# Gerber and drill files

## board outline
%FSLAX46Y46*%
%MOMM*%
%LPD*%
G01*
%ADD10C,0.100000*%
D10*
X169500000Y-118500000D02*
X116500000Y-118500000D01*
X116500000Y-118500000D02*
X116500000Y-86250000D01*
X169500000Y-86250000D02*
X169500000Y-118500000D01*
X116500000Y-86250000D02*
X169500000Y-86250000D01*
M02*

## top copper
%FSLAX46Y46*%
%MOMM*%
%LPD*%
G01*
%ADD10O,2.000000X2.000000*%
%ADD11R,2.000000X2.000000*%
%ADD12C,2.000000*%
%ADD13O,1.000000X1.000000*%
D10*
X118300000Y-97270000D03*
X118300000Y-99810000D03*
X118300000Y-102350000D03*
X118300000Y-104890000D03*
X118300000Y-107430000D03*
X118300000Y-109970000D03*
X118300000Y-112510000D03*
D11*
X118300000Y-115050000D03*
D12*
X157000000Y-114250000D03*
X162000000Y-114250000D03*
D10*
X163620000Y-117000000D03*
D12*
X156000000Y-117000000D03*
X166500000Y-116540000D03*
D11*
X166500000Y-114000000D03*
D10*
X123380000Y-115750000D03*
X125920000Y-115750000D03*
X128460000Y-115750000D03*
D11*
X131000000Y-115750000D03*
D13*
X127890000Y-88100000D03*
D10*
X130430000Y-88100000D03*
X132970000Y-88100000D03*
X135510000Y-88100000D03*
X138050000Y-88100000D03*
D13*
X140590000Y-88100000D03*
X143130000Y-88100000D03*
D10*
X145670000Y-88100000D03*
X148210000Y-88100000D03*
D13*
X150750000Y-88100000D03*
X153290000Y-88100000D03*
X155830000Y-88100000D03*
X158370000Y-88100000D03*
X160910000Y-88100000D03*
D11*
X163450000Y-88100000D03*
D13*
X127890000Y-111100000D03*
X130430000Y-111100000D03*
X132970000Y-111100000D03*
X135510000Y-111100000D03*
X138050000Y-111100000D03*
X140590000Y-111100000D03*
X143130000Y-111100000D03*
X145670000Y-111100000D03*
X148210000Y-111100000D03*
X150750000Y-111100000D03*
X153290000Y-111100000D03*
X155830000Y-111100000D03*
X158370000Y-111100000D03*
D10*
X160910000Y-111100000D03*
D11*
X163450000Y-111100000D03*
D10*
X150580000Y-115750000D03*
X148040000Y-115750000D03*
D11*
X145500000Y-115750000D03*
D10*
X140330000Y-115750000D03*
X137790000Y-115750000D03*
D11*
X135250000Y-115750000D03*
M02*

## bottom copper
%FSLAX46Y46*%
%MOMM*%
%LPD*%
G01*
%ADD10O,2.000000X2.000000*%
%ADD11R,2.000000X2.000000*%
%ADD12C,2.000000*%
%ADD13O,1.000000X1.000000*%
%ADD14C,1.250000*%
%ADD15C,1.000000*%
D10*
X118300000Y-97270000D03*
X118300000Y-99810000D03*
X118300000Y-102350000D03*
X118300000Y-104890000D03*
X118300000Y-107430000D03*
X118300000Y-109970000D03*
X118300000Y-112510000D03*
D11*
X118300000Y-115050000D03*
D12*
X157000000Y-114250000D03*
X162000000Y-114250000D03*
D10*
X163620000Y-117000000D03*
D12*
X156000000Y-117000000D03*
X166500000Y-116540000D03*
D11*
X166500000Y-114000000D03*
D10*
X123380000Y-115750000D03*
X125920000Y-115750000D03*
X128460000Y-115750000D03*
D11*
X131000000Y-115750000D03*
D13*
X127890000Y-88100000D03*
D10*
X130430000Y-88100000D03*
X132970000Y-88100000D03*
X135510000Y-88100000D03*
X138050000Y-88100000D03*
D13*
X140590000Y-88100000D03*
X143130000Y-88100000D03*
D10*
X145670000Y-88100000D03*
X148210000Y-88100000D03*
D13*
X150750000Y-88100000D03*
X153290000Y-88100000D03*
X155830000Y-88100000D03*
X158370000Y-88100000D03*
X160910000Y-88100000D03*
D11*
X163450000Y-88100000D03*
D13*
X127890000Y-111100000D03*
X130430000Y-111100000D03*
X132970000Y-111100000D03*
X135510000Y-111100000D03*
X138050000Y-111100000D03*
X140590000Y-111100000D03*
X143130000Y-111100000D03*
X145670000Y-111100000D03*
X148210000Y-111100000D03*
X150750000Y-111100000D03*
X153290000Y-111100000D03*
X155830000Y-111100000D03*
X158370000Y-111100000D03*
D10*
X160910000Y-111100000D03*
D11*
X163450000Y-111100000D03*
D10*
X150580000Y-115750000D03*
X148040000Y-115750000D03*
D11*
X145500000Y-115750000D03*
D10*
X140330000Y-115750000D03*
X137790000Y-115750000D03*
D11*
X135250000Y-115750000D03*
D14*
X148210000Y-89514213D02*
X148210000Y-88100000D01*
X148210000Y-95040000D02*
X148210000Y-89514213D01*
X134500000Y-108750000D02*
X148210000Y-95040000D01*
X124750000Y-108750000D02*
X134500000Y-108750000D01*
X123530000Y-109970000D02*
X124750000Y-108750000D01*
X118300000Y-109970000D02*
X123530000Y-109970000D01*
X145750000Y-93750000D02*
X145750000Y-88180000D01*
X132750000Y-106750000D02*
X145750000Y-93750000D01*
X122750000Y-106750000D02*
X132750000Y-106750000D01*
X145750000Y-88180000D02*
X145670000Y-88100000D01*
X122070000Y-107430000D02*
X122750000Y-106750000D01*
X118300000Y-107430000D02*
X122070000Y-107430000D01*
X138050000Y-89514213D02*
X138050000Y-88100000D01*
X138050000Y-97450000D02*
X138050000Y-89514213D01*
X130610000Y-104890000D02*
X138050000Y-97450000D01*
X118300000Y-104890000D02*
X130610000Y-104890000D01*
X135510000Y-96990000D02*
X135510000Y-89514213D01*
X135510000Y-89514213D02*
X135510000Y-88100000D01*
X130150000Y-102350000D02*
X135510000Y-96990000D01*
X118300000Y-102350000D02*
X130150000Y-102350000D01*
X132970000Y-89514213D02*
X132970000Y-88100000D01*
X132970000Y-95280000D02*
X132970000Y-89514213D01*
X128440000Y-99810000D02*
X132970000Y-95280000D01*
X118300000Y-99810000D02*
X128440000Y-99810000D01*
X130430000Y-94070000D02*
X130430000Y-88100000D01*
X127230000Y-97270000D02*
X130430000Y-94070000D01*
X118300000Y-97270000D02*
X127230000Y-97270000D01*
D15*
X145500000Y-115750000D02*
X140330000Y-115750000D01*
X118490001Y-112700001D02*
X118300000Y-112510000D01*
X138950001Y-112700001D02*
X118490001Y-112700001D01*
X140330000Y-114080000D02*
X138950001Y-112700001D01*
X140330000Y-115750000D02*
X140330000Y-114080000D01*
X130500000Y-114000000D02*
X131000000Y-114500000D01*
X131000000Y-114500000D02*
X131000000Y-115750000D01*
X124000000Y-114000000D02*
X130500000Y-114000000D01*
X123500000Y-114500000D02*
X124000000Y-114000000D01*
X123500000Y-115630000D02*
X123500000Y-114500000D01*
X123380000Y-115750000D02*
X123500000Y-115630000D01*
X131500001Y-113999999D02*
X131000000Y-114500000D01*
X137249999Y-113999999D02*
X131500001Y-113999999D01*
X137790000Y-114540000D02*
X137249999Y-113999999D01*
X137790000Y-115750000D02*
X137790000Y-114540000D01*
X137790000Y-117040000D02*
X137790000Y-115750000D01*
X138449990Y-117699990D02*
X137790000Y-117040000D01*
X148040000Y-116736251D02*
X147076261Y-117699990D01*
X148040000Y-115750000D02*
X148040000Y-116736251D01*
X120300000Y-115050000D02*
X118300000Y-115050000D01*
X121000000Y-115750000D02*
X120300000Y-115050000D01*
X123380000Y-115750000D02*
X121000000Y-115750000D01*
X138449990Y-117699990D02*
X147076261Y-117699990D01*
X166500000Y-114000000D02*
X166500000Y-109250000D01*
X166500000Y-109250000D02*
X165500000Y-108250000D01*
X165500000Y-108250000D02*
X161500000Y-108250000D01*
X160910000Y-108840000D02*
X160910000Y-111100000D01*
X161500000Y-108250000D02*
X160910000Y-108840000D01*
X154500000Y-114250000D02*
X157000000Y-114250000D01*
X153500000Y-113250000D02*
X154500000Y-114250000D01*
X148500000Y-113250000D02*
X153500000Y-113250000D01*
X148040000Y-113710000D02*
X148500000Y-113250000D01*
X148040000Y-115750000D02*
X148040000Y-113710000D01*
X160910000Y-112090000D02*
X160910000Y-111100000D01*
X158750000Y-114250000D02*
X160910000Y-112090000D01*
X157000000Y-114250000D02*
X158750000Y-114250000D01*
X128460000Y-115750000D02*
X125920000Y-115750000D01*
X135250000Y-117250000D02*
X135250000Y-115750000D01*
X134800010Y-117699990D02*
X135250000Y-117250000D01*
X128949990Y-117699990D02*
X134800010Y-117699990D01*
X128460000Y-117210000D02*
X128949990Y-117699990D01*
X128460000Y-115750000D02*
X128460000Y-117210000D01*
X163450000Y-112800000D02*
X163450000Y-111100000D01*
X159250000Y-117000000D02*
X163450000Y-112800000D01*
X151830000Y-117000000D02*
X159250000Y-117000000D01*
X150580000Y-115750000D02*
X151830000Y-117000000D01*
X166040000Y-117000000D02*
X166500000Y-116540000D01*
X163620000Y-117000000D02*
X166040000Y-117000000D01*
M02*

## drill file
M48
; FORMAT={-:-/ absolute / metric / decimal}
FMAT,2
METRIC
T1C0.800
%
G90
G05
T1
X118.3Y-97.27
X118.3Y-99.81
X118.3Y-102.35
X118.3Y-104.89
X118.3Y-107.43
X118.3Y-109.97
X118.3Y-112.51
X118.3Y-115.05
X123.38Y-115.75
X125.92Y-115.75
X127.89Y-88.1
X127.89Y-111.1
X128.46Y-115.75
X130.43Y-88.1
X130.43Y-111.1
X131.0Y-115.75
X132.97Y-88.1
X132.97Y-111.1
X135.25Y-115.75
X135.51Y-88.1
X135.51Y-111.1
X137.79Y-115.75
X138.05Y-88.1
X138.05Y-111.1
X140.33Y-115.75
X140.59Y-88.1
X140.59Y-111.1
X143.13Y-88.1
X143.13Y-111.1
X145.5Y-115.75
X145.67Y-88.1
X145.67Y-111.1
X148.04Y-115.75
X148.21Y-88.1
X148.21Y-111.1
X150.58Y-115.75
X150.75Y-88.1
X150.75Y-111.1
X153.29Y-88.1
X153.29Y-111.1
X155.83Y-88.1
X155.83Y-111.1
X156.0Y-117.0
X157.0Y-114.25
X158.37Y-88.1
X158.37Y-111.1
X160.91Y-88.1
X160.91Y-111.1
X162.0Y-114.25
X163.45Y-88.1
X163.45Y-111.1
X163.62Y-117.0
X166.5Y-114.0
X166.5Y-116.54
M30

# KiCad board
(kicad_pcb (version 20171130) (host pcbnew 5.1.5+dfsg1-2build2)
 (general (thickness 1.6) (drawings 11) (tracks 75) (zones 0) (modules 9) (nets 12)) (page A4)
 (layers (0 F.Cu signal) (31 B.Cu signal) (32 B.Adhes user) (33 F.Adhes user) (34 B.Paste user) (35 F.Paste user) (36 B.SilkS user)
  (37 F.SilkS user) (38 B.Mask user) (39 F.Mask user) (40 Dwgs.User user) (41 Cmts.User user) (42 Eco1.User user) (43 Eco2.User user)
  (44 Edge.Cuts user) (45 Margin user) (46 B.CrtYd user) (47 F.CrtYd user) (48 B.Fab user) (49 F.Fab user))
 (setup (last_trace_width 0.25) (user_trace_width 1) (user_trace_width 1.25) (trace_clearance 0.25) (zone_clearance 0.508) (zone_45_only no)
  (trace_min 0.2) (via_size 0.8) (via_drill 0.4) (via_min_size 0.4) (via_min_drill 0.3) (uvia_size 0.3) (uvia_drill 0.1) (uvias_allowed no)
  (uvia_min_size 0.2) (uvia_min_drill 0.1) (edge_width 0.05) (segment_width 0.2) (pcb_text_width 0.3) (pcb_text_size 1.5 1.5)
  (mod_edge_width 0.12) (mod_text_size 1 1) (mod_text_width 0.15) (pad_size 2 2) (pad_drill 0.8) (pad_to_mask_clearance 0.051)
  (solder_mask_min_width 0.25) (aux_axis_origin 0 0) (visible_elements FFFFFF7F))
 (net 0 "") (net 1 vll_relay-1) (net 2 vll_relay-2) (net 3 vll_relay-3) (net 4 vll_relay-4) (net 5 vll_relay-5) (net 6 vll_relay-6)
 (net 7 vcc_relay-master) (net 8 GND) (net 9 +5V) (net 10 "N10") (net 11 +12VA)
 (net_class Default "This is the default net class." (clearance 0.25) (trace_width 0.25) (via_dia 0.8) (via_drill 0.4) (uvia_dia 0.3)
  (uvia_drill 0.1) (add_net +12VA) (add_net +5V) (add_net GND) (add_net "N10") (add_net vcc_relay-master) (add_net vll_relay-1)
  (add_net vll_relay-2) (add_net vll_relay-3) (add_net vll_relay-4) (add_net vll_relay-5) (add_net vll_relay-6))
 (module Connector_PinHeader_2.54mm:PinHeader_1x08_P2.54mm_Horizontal (layer F.Cu) (at 118.3 115.05 180)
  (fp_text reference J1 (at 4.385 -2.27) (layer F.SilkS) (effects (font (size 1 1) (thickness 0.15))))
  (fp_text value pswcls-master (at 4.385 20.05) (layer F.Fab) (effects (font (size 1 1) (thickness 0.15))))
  (pad 8 thru_hole oval (at 0 17.78 180) (size 2 2) (drill 0.8) (layers *.Cu *.Mask) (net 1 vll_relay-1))
  (pad 7 thru_hole oval (at 0 15.24 180) (size 2 2) (drill 0.8) (layers *.Cu *.Mask) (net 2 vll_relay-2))
  (pad 6 thru_hole oval (at 0 12.7 180) (size 2 2) (drill 0.8) (layers *.Cu *.Mask) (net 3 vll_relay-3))
  (pad 5 thru_hole oval (at 0 10.16 180) (size 2 2) (drill 0.8) (layers *.Cu *.Mask) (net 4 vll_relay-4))
  (pad 4 thru_hole oval (at 0 7.62 180) (size 2 2) (drill 0.8) (layers *.Cu *.Mask) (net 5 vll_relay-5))
  (pad 3 thru_hole oval (at 0 5.08 180) (size 2 2) (drill 0.8) (layers *.Cu *.Mask) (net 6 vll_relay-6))
  (pad 2 thru_hole oval (at 0 2.54 180) (size 2 2) (drill 0.8) (layers *.Cu *.Mask) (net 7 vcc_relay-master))
  (pad 1 thru_hole rect (at 0 0 180) (size 2 2) (drill 0.8) (layers *.Cu *.Mask) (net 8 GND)))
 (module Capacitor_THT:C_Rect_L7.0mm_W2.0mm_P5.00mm (layer F.Cu) (at 162 114.25 180)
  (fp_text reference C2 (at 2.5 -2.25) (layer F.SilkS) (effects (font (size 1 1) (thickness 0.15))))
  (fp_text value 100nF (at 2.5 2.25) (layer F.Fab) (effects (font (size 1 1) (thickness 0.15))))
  (pad 2 thru_hole circle (at 5 0 180) (size 2 2) (drill 0.8) (layers *.Cu *.Mask) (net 8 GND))
  (pad 1 thru_hole circle (at 0 0 180) (size 2 2) (drill 0.8) (layers *.Cu *.Mask) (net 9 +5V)))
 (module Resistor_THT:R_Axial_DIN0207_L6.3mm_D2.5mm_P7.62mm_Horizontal (layer F.Cu) (at 156 117)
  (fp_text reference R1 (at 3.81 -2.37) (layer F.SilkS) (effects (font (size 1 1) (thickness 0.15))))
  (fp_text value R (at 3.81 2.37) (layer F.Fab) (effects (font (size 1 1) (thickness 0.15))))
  (pad 2 thru_hole oval (at 7.62 0) (size 2 2) (drill 0.8) (layers *.Cu *.Mask) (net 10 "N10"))
  (pad 1 thru_hole circle (at 0 0) (size 2 2) (drill 0.8) (layers *.Cu *.Mask) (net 9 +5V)))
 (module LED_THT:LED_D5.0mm (layer F.Cu) (at 166.5 114 270)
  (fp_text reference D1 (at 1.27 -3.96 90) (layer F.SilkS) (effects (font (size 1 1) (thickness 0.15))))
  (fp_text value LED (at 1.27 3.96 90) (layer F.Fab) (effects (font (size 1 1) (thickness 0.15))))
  (pad 2 thru_hole circle (at 2.54 0 270) (size 2 2) (drill 0.8) (layers *.Cu *.Mask) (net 10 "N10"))
  (pad 1 thru_hole rect (at 0 0 270) (size 2 2) (drill 0.8) (layers *.Cu *.Mask) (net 8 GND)))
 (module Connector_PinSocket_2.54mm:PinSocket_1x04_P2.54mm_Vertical (layer F.Cu) (at 131 115.75 270)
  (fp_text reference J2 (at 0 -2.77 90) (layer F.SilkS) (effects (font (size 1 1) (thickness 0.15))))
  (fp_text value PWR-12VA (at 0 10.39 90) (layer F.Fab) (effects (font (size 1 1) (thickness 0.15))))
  (pad 4 thru_hole oval (at 0 7.62 270) (size 2 2) (drill 0.8) (layers *.Cu *.Mask) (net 8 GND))
  (pad 3 thru_hole oval (at 0 5.08 270) (size 2 2) (drill 0.8) (layers *.Cu *.Mask) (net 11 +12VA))
  (pad 2 thru_hole oval (at 0 2.54 270) (size 2 2) (drill 0.8) (layers *.Cu *.Mask) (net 11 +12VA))
  (pad 1 thru_hole rect (at 0 0 270) (size 2 2) (drill 0.8) (layers *.Cu *.Mask) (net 8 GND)))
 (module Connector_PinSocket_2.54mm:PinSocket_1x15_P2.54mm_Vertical (layer F.Cu) (at 163.45 88.1 270)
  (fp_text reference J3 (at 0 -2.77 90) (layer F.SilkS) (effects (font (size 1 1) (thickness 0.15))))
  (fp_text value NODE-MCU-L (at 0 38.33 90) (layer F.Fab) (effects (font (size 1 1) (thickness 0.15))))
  (pad 15 thru_hole oval (at 0 35.56 270) (size 1 1) (drill 0.8) (layers *.Cu *.Mask))
  (pad 14 thru_hole oval (at 0 33.02 270) (size 2 2) (drill 0.8) (layers *.Cu *.Mask) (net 1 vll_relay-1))
  (pad 13 thru_hole oval (at 0 30.48 270) (size 2 2) (drill 0.8) (layers *.Cu *.Mask) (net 2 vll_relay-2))
  (pad 12 thru_hole oval (at 0 27.94 270) (size 2 2) (drill 0.8) (layers *.Cu *.Mask) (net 3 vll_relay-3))
  (pad 11 thru_hole oval (at 0 25.4 270) (size 2 2) (drill 0.8) (layers *.Cu *.Mask) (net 4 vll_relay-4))
  (pad 10 thru_hole oval (at 0 22.86 270) (size 1 1) (drill 0.8) (layers *.Cu *.Mask))
  (pad 9 thru_hole oval (at 0 20.32 270) (size 1 1) (drill 0.8) (layers *.Cu *.Mask))
  (pad 8 thru_hole oval (at 0 17.78 270) (size 2 2) (drill 0.8) (layers *.Cu *.Mask) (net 5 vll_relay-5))
  (pad 7 thru_hole oval (at 0 15.24 270) (size 2 2) (drill 0.8) (layers *.Cu *.Mask) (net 6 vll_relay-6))
  (pad 6 thru_hole oval (at 0 12.7 270) (size 1 1) (drill 0.8) (layers *.Cu *.Mask))
  (pad 5 thru_hole oval (at 0 10.16 270) (size 1 1) (drill 0.8) (layers *.Cu *.Mask))
  (pad 4 thru_hole oval (at 0 7.62 270) (size 1 1) (drill 0.8) (layers *.Cu *.Mask))
  (pad 3 thru_hole oval (at 0 5.08 270) (size 1 1) (drill 0.8) (layers *.Cu *.Mask))
  (pad 2 thru_hole oval (at 0 2.54 270) (size 1 1) (drill 0.8) (layers *.Cu *.Mask))
  (pad 1 thru_hole rect (at 0 0 270) (size 2 2) (drill 0.8) (layers *.Cu *.Mask)))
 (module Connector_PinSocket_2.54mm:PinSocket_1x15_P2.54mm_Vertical (layer F.Cu) (at 163.45 111.1 270)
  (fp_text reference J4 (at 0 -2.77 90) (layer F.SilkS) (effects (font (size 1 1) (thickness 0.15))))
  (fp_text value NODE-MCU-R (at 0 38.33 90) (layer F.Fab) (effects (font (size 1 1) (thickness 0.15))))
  (pad 15 thru_hole oval (at 0 35.56 270) (size 1 1) (drill 0.8) (layers *.Cu *.Mask))
  (pad 14 thru_hole oval (at 0 33.02 270) (size 1 1) (drill 0.8) (layers *.Cu *.Mask))
  (pad 13 thru_hole oval (at 0 30.48 270) (size 1 1) (drill 0.8) (layers *.Cu *.Mask))
  (pad 12 thru_hole oval (at 0 27.94 270) (size 1 1) (drill 0.8) (layers *.Cu *.Mask))
  (pad 11 thru_hole oval (at 0 25.4 270) (size 1 1) (drill 0.8) (layers *.Cu *.Mask))
  (pad 10 thru_hole oval (at 0 22.86 270) (size 1 1) (drill 0.8) (layers *.Cu *.Mask))
  (pad 9 thru_hole oval (at 0 20.32 270) (size 1 1) (drill 0.8) (layers *.Cu *.Mask))
  (pad 8 thru_hole oval (at 0 17.78 270) (size 1 1) (drill 0.8) (layers *.Cu *.Mask))
  (pad 7 thru_hole oval (at 0 15.24 270) (size 1 1) (drill 0.8) (layers *.Cu *.Mask))
  (pad 6 thru_hole oval (at 0 12.7 270) (size 1 1) (drill 0.8) (layers *.Cu *.Mask))
  (pad 5 thru_hole oval (at 0 10.16 270) (size 1 1) (drill 0.8) (layers *.Cu *.Mask))
  (pad 4 thru_hole oval (at 0 7.62 270) (size 1 1) (drill 0.8) (layers *.Cu *.Mask))
  (pad 3 thru_hole oval (at 0 5.08 270) (size 1 1) (drill 0.8) (layers *.Cu *.Mask))
  (pad 2 thru_hole oval (at 0 2.54 270) (size 2 2) (drill 0.8) (layers *.Cu *.Mask) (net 8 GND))
  (pad 1 thru_hole rect (at 0 0 270) (size 2 2) (drill 0.8) (layers *.Cu *.Mask) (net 9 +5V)))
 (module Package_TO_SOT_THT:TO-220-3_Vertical (layer F.Cu) (at 145.5 115.75)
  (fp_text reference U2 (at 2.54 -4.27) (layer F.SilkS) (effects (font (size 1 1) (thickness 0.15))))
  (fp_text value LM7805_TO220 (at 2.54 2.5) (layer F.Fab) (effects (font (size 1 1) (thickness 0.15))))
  (pad 3 thru_hole oval (at 5.08 0) (size 2 2) (drill 0.8) (layers *.Cu *.Mask) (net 9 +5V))
  (pad 2 thru_hole oval (at 2.54 0) (size 2 2) (drill 0.8) (layers *.Cu *.Mask) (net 8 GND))
  (pad 1 thru_hole rect (at 0 0) (size 2 2) (drill 0.8) (layers *.Cu *.Mask) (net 7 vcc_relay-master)))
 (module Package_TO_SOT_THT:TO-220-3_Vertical (layer F.Cu) (at 135.25 115.75)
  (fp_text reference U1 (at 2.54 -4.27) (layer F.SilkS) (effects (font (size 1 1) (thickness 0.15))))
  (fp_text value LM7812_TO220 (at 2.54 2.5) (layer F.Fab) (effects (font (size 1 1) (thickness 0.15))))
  (pad 3 thru_hole oval (at 5.08 0) (size 2 2) (drill 0.8) (layers *.Cu *.Mask) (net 7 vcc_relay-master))
  (pad 2 thru_hole oval (at 2.54 0) (size 2 2) (drill 0.8) (layers *.Cu *.Mask) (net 8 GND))
  (pad 1 thru_hole rect (at 0 0) (size 2 2) (drill 0.8) (layers *.Cu *.Mask) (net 11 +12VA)))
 (gr_line (start 169.5 118.5) (end 116.5 118.5) (layer Edge.Cuts) (width 0.1))
 (gr_line (start 116.5 118.5) (end 116.5 86.25) (layer Edge.Cuts) (width 0.1))
 (gr_line (start 169.5 86.25) (end 169.5 118.5) (layer Edge.Cuts) (width 0.1))
 (gr_line (start 116.5 86.25) (end 169.5 86.25) (layer Edge.Cuts) (width 0.1))
 (segment (start 148.21 89.514213) (end 148.21 88.1) (width 1.25) (layer B.Cu) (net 6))
 (segment (start 148.21 95.04) (end 148.21 89.514213) (width 1.25) (layer B.Cu) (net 6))
 (segment (start 134.5 108.75) (end 148.21 95.04) (width 1.25) (layer B.Cu) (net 6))
 (segment (start 124.75 108.75) (end 134.5 108.75) (width 1.25) (layer B.Cu) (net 6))
 (segment (start 123.53 109.97) (end 124.75 108.75) (width 1.25) (layer B.Cu) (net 6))
 (segment (start 118.3 109.97) (end 123.53 109.97) (width 1.25) (layer B.Cu) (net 6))
 (segment (start 145.75 93.75) (end 145.75 88.18) (width 1.25) (layer B.Cu) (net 5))
 (segment (start 132.75 106.75) (end 145.75 93.75) (width 1.25) (layer B.Cu) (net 5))
 (segment (start 122.75 106.75) (end 132.75 106.75) (width 1.25) (layer B.Cu) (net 5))
 (segment (start 145.75 88.18) (end 145.67 88.1) (width 1.25) (layer B.Cu) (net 5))
 (segment (start 122.07 107.43) (end 122.75 106.75) (width 1.25) (layer B.Cu) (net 5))
 (segment (start 118.3 107.43) (end 122.07 107.43) (width 1.25) (layer B.Cu) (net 5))
 (segment (start 138.05 89.514213) (end 138.05 88.1) (width 1.25) (layer B.Cu) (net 4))
 (segment (start 138.05 97.45) (end 138.05 89.514213) (width 1.25) (layer B.Cu) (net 4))
 (segment (start 130.61 104.89) (end 138.05 97.45) (width 1.25) (layer B.Cu) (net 4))
 (segment (start 118.3 104.89) (end 130.61 104.89) (width 1.25) (layer B.Cu) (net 4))
 (segment (start 135.51 96.99) (end 135.51 89.514213) (width 1.25) (layer B.Cu) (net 3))
 (segment (start 135.51 89.514213) (end 135.51 88.1) (width 1.25) (layer B.Cu) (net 3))
 (segment (start 130.15 102.35) (end 135.51 96.99) (width 1.25) (layer B.Cu) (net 3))
 (segment (start 118.3 102.35) (end 130.15 102.35) (width 1.25) (layer B.Cu) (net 3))
 (segment (start 132.97 89.514213) (end 132.97 88.1) (width 1.25) (layer B.Cu) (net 2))
 (segment (start 132.97 95.28) (end 132.97 89.514213) (width 1.25) (layer B.Cu) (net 2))
 (segment (start 128.44 99.81) (end 132.97 95.28) (width 1.25) (layer B.Cu) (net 2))
 (segment (start 118.3 99.81) (end 128.44 99.81) (width 1.25) (layer B.Cu) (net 2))
 (segment (start 130.43 94.07) (end 130.43 88.1) (width 1.25) (layer B.Cu) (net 1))
 (segment (start 127.23 97.27) (end 130.43 94.07) (width 1.25) (layer B.Cu) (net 1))
 (segment (start 118.3 97.27) (end 127.23 97.27) (width 1.25) (layer B.Cu) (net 1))
 (segment (start 145.5 115.75) (end 140.33 115.75) (width 1) (layer B.Cu) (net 7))
 (segment (start 118.490001 112.700001) (end 118.3 112.51) (width 1) (layer B.Cu) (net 7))
 (segment (start 138.950001 112.700001) (end 118.490001 112.700001) (width 1) (layer B.Cu) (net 7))
 (segment (start 140.33 114.08) (end 138.950001 112.700001) (width 1) (layer B.Cu) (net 7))
 (segment (start 140.33 115.75) (end 140.33 114.08) (width 1) (layer B.Cu) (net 7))
 (segment (start 130.5 114) (end 131 114.5) (width 1) (layer B.Cu) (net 8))
 (segment (start 131 114.5) (end 131 115.75) (width 1) (layer B.Cu) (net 8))
 (segment (start 124 114) (end 130.5 114) (width 1) (layer B.Cu) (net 8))
 (segment (start 123.5 114.5) (end 124 114) (width 1) (layer B.Cu) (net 8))
 (segment (start 123.5 115.63) (end 123.5 114.5) (width 1) (layer B.Cu) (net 8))
 (segment (start 123.38 115.75) (end 123.5 115.63) (width 1) (layer B.Cu) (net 8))
 (segment (start 131.500001 113.999999) (end 131 114.5) (width 1) (layer B.Cu) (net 8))
 (segment (start 137.249999 113.999999) (end 131.500001 113.999999) (width 1) (layer B.Cu) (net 8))
 (segment (start 137.79 114.54) (end 137.249999 113.999999) (width 1) (layer B.Cu) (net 8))
 (segment (start 137.79 115.75) (end 137.79 114.54) (width 1) (layer B.Cu) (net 8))
 (segment (start 137.79 117.04) (end 137.79 115.75) (width 1) (layer B.Cu) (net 8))
 (segment (start 138.44999 117.69999) (end 137.79 117.04) (width 1) (layer B.Cu) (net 8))
 (segment (start 148.04 116.736251) (end 147.076261 117.69999) (width 1) (layer B.Cu) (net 8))
 (segment (start 148.04 115.75) (end 148.04 116.736251) (width 1) (layer B.Cu) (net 8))
 (segment (start 120.3 115.05) (end 118.3 115.05) (width 1) (layer B.Cu) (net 8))
 (segment (start 121 115.75) (end 120.3 115.05) (width 1) (layer B.Cu) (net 8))
 (segment (start 123.38 115.75) (end 121 115.75) (width 1) (layer B.Cu) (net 8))
 (segment (start 138.44999 117.69999) (end 147.076261 117.69999) (width 1) (layer B.Cu) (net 8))
 (segment (start 166.5 114) (end 166.5 109.25) (width 1) (layer B.Cu) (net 8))
 (segment (start 166.5 109.25) (end 165.5 108.25) (width 1) (layer B.Cu) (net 8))
 (segment (start 165.5 108.25) (end 161.5 108.25) (width 1) (layer B.Cu) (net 8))
 (segment (start 160.91 108.84) (end 160.91 111.1) (width 1) (layer B.Cu) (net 8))
 (segment (start 161.5 108.25) (end 160.91 108.84) (width 1) (layer B.Cu) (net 8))
 (segment (start 154.5 114.25) (end 157 114.25) (width 1) (layer B.Cu) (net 8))
 (segment (start 153.5 113.25) (end 154.5 114.25) (width 1) (layer B.Cu) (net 8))
 (segment (start 148.5 113.25) (end 153.5 113.25) (width 1) (layer B.Cu) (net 8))
 (segment (start 148.04 113.71) (end 148.5 113.25) (width 1) (layer B.Cu) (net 8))
 (segment (start 148.04 115.75) (end 148.04 113.71) (width 1) (layer B.Cu) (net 8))
 (segment (start 160.91 112.09) (end 160.91 111.1) (width 1) (layer B.Cu) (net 8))
 (segment (start 158.75 114.25) (end 160.91 112.09) (width 1) (layer B.Cu) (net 8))
 (segment (start 157 114.25) (end 158.75 114.25) (width 1) (layer B.Cu) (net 8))
 (segment (start 128.46 115.75) (end 125.92 115.75) (width 1) (layer B.Cu) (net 11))
 (segment (start 135.25 117.25) (end 135.25 115.75) (width 1) (layer B.Cu) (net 11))
 (segment (start 134.80001 117.69999) (end 135.25 117.25) (width 1) (layer B.Cu) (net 11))
 (segment (start 128.94999 117.69999) (end 134.80001 117.69999) (width 1) (layer B.Cu) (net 11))
 (segment (start 128.46 117.21) (end 128.94999 117.69999) (width 1) (layer B.Cu) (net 11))
 (segment (start 128.46 115.75) (end 128.46 117.21) (width 1) (layer B.Cu) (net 11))
 (segment (start 163.45 112.8) (end 163.45 111.1) (width 1) (layer B.Cu) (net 9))
 (segment (start 159.25 117) (end 163.45 112.8) (width 1) (layer B.Cu) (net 9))
 (segment (start 151.83 117) (end 159.25 117) (width 1) (layer B.Cu) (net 9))
 (segment (start 150.58 115.75) (end 151.83 117) (width 1) (layer B.Cu) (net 9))
 (segment (start 166.04 117) (end 166.5 116.54) (width 1) (layer B.Cu) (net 10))
 (segment (start 163.62 117) (end 166.04 117) (width 1) (layer B.Cu) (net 10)))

